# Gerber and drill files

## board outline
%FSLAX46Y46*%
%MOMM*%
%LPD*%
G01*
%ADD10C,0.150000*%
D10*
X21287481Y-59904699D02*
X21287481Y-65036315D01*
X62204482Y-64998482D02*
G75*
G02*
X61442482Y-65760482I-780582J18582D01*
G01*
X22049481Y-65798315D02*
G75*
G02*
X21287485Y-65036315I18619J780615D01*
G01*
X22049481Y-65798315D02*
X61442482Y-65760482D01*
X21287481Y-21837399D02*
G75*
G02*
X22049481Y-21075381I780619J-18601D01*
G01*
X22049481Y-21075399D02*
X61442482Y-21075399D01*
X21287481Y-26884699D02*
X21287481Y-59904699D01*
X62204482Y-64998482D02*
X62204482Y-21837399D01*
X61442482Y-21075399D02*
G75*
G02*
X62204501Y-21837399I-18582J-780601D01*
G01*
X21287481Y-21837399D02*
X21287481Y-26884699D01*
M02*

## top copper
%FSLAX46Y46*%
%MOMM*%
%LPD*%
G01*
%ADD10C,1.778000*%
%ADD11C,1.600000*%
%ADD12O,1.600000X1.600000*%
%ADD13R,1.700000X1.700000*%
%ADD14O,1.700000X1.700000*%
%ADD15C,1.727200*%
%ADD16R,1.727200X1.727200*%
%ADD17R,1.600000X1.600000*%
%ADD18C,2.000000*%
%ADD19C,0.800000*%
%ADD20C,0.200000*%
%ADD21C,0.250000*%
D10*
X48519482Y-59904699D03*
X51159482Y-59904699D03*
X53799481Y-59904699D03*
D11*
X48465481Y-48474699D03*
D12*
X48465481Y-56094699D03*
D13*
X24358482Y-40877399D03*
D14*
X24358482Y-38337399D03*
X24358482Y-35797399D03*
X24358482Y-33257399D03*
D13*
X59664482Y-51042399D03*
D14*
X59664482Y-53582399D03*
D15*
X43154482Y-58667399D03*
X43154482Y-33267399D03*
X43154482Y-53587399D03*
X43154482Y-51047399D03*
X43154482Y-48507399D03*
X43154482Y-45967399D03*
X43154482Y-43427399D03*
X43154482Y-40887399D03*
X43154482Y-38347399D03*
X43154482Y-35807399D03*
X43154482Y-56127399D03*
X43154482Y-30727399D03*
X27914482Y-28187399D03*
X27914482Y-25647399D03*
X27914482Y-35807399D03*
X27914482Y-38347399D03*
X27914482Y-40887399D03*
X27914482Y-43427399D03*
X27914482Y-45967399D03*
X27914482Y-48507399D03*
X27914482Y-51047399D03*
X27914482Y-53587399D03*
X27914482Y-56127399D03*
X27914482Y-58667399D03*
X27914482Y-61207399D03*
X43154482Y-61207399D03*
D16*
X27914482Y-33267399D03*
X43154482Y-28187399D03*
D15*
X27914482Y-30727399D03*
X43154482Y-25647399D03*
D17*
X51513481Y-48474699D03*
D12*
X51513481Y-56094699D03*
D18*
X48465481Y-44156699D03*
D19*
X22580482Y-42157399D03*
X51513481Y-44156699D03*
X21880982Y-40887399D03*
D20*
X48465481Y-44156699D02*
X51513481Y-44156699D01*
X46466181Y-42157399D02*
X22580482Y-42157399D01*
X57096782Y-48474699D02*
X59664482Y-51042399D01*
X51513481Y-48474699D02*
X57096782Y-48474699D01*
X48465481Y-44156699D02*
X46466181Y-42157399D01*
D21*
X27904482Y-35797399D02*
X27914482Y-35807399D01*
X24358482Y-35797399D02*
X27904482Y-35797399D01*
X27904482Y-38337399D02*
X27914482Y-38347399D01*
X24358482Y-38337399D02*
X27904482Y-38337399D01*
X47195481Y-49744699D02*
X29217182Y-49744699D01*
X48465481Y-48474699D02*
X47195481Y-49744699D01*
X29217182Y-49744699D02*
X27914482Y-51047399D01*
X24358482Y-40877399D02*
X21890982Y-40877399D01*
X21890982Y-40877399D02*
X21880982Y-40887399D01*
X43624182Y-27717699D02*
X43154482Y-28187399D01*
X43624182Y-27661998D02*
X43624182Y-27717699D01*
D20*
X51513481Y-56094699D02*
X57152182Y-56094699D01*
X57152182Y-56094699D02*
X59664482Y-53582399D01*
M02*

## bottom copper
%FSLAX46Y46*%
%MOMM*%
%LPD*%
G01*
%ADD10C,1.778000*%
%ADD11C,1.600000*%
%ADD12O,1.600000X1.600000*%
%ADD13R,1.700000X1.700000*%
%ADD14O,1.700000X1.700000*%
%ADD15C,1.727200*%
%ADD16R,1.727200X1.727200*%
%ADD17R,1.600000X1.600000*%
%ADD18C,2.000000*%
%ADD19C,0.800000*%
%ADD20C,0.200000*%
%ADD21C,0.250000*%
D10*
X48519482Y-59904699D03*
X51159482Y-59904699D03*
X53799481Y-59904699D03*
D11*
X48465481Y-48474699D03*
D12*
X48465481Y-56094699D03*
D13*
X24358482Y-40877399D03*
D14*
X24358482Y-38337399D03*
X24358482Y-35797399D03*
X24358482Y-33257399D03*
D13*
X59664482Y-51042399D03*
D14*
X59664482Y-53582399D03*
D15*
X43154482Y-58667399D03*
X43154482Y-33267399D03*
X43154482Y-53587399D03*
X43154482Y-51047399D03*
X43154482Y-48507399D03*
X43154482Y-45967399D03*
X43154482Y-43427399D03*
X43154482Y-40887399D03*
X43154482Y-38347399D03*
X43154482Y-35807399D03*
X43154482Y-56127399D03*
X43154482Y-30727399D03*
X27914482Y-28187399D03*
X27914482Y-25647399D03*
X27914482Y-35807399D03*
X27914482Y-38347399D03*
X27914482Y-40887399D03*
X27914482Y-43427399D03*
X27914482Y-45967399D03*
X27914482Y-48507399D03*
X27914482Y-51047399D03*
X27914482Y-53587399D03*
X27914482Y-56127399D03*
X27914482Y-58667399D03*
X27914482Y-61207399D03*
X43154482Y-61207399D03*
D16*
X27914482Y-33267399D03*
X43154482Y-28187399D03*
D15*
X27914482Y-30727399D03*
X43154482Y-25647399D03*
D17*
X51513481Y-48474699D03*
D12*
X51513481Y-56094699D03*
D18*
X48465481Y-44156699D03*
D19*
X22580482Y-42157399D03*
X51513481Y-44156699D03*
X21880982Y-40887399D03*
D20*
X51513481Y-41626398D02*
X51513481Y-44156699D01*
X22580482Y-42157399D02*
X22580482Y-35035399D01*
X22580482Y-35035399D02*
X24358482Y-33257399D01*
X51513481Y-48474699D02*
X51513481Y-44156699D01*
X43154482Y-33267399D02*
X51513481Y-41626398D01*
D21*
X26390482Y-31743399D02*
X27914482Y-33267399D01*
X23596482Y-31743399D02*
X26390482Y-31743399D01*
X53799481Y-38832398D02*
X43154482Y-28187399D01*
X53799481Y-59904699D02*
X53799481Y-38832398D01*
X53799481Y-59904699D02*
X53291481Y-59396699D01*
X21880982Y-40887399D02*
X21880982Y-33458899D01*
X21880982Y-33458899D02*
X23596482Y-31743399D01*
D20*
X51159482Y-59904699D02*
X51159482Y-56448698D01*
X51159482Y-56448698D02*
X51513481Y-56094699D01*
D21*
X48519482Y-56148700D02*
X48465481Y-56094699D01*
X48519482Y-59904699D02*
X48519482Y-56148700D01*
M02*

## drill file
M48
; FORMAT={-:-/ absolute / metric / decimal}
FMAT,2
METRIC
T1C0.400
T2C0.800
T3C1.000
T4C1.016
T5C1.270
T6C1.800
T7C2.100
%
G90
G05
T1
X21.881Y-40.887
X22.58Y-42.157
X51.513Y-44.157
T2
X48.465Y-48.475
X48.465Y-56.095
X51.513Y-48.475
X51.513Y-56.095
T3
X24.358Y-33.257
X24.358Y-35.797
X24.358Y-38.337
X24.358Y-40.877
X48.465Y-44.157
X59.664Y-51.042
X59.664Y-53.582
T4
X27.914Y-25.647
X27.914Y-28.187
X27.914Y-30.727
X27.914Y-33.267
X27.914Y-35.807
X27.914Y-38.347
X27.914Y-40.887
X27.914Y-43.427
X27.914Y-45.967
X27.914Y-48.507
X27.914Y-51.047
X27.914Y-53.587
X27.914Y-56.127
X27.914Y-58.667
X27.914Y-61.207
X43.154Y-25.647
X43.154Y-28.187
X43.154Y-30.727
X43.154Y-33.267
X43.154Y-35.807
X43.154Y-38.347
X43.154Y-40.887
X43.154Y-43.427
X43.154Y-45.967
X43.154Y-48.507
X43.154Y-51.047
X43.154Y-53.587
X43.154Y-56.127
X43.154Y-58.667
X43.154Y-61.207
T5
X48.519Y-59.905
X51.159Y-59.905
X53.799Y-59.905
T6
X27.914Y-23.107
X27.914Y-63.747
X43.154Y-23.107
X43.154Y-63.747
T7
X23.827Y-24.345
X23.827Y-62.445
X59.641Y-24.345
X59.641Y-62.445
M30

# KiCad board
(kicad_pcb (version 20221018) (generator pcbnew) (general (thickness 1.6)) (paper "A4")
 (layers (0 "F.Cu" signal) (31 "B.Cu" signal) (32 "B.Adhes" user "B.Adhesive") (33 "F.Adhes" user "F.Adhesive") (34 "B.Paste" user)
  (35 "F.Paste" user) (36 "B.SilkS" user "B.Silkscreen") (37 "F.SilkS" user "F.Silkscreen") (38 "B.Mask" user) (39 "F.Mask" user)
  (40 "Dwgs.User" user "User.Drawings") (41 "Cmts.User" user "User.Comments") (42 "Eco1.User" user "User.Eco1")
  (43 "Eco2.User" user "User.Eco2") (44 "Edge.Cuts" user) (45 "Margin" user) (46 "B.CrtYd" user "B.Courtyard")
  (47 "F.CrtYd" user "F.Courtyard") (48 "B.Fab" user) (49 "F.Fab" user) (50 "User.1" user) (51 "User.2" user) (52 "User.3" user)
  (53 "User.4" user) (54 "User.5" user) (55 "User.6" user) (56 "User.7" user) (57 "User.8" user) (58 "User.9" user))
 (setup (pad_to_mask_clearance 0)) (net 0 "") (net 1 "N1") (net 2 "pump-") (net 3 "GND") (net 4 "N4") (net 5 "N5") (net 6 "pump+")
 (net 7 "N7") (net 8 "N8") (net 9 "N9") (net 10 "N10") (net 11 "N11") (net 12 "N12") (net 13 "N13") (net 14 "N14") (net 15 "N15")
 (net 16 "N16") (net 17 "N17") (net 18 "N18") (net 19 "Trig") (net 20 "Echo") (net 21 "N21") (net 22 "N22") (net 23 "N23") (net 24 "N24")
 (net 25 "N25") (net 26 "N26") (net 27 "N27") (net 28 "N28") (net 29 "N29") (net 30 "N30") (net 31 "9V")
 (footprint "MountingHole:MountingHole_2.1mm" (layer "F.Cu") (at 59.641481 62.444699)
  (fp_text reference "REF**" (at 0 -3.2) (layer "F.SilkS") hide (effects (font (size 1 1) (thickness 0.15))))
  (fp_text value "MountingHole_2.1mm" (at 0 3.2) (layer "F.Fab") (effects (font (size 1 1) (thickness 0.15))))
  (pad "" np_thru_hole circle (at 0 0) (size 2.1 2.1) (drill 2.1) (layers "F&B.Cu" "*.Mask")))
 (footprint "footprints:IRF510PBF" (layer "F.Cu") (at 48.519482 59.904699)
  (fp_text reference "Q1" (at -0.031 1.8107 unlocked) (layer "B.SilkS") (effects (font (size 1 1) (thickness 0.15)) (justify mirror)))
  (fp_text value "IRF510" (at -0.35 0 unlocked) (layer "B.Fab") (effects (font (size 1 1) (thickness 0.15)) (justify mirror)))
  (pad "1" thru_hole circle (at 0 0) (size 1.778 1.778) (drill 1.27) (layers "*.Cu" "*.Mask") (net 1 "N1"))
  (pad "2" thru_hole circle (at 2.64 0) (size 1.778 1.778) (drill 1.27) (layers "*.Cu" "*.Mask") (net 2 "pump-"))
  (pad "3" thru_hole circle (at 5.279999 0) (size 1.778 1.778) (drill 1.27) (layers "*.Cu" "*.Mask") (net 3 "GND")))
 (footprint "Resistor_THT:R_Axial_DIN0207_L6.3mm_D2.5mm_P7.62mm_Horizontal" (layer "F.Cu") (at 48.465481 48.474699 -90)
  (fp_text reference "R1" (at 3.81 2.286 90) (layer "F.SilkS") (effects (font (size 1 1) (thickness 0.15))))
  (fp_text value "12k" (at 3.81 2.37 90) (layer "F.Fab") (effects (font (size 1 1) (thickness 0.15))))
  (pad "1" thru_hole circle (at 0 0 270) (size 1.6 1.6) (drill 0.8) (layers "*.Cu" "*.Mask") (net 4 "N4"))
  (pad "2" thru_hole oval (at 7.62 0 270) (size 1.6 1.6) (drill 0.8) (layers "*.Cu" "*.Mask") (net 1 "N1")))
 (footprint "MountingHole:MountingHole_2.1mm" (layer "F.Cu") (at 23.827481 62.444699)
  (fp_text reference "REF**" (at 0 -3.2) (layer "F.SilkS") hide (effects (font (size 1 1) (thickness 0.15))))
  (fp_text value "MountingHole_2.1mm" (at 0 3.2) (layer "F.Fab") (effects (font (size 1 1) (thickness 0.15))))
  (pad "" np_thru_hole circle (at 0 0) (size 2.1 2.1) (drill 2.1) (layers "F&B.Cu" "*.Mask")))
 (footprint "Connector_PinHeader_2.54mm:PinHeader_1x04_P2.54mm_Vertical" (layer "F.Cu") (at 24.358482 40.877399 180)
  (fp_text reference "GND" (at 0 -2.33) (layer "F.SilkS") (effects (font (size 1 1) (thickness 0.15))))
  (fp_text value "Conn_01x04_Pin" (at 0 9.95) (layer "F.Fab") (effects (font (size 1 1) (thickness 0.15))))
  (pad "1" thru_hole rect (at 0 0 180) (size 1.7 1.7) (drill 1) (layers "*.Cu" "*.Mask"))
  (pad "2" thru_hole oval (at 0 2.54 180) (size 1.7 1.7) (drill 1) (layers "*.Cu" "*.Mask"))
  (pad "3" thru_hole oval (at 0 5.08 180) (size 1.7 1.7) (drill 1) (layers "*.Cu" "*.Mask"))
  (pad "4" thru_hole oval (at 0 7.62 180) (size 1.7 1.7) (drill 1) (layers "*.Cu" "*.Mask")))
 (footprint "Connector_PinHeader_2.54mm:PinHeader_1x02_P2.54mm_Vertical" (layer "F.Cu") (at 59.664482 51.042399)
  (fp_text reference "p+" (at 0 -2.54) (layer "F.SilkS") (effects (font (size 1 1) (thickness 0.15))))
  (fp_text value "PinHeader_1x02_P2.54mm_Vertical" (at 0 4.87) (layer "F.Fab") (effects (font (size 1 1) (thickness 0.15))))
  (pad "1" thru_hole rect (at 0 0) (size 1.7 1.7) (drill 1) (layers "*.Cu" "*.Mask"))
  (pad "2" thru_hole oval (at 0 2.54) (size 1.7 1.7) (drill 1) (layers "*.Cu" "*.Mask")))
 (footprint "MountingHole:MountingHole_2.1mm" (layer "F.Cu") (at 59.641481 24.344699)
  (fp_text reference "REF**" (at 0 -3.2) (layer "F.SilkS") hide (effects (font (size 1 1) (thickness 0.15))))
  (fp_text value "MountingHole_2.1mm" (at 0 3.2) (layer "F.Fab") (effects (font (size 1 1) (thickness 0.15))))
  (pad "" np_thru_hole circle (at 0 0) (size 2.1 2.1) (drill 2.1) (layers "F&B.Cu" "*.Mask")))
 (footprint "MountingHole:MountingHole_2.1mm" (layer "F.Cu") (at 23.827481 24.344699)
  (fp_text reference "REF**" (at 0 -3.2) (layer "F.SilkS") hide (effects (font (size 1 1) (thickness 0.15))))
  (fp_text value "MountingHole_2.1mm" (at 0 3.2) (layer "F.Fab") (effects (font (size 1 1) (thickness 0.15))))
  (pad "" np_thru_hole circle (at 0 0) (size 2.1 2.1) (drill 2.1) (layers "F&B.Cu" "*.Mask")))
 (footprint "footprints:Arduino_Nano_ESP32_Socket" (layer "F.Cu") (at 35.534482 65.017399)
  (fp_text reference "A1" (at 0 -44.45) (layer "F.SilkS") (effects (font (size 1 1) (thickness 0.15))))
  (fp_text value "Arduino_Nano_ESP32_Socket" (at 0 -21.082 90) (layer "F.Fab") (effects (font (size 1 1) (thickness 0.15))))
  (pad "" np_thru_hole circle (at -7.62 -41.91) (size 1.8 1.8) (drill 1.8) (layers "F&B.Cu" "*.Mask"))
  (pad "" np_thru_hole circle (at -7.62 -1.27) (size 1.8 1.8) (drill 1.8) (layers "F&B.Cu" "*.Mask"))
  (pad "" np_thru_hole circle (at 7.62 -41.91) (size 1.8 1.8) (drill 1.8) (layers "F&B.Cu" "*.Mask"))
  (pad "" np_thru_hole circle (at 7.62 -1.27) (size 1.8 1.8) (drill 1.8) (layers "F&B.Cu" "*.Mask"))
  (pad "3V3" thru_hole circle (at 7.62 -6.35) (size 1.7272 1.7272) (drill 1.016) (layers "*.Cu" "*.Mask") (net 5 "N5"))
  (pad "5V" thru_hole circle (at 7.62 -31.75) (size 1.7272 1.7272) (drill 1.016) (layers "*.Cu" "*.Mask") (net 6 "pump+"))
  (pad "A0" thru_hole circle (at 7.62 -11.43) (size 1.7272 1.7272) (drill 1.016) (layers "*.Cu" "*.Mask") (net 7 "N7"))
  (pad "A1" thru_hole circle (at 7.62 -13.97) (size 1.7272 1.7272) (drill 1.016) (layers "*.Cu" "*.Mask") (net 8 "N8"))
  (pad "A2" thru_hole circle (at 7.62 -16.51) (size 1.7272 1.7272) (drill 1.016) (layers "*.Cu" "*.Mask") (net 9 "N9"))
  (pad "A3" thru_hole circle (at 7.62 -19.05) (size 1.7272 1.7272) (drill 1.016) (layers "*.Cu" "*.Mask") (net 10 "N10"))
  (pad "A4" thru_hole circle (at 7.62 -21.59) (size 1.7272 1.7272) (drill 1.016) (layers "*.Cu" "*.Mask") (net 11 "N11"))
  (pad "A5" thru_hole circle (at 7.62 -24.13) (size 1.7272 1.7272) (drill 1.016) (layers "*.Cu" "*.Mask") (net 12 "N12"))
  (pad "A6" thru_hole circle (at 7.62 -26.67) (size 1.7272 1.7272) (drill 1.016) (layers "*.Cu" "*.Mask") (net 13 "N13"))
  (pad "A7" thru_hole circle (at 7.62 -29.21) (size 1.7272 1.7272) (drill 1.016) (layers "*.Cu" "*.Mask") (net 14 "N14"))
  (pad "B0" thru_hole circle (at 7.62 -8.89) (size 1.7272 1.7272) (drill 1.016) (layers "*.Cu" "*.Mask") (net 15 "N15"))
  (pad "B1" thru_hole circle (at 7.62 -34.29) (size 1.7272 1.7272) (drill 1.016) (layers "*.Cu" "*.Mask") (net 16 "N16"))
  (pad "D0" thru_hole circle (at -7.62 -36.83) (size 1.7272 1.7272) (drill 1.016) (layers "*.Cu" "*.Mask") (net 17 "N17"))
  (pad "D1" thru_hole circle (at -7.62 -39.37) (size 1.7272 1.7272) (drill 1.016) (layers "*.Cu" "*.Mask") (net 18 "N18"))
  (pad "D2" thru_hole circle (at -7.62 -29.21) (size 1.7272 1.7272) (drill 1.016) (layers "*.Cu" "*.Mask") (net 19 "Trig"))
  (pad "D3" thru_hole circle (at -7.62 -26.67) (size 1.7272 1.7272) (drill 1.016) (layers "*.Cu" "*.Mask") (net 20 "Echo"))
  (pad "D4" thru_hole circle (at -7.62 -24.13) (size 1.7272 1.7272) (drill 1.016) (layers "*.Cu" "*.Mask") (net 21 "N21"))
  (pad "D5" thru_hole circle (at -7.62 -21.59) (size 1.7272 1.7272) (drill 1.016) (layers "*.Cu" "*.Mask") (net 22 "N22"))
  (pad "D6" thru_hole circle (at -7.62 -19.05) (size 1.7272 1.7272) (drill 1.016) (layers "*.Cu" "*.Mask") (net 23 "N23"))
  (pad "D7" thru_hole circle (at -7.62 -16.51) (size 1.7272 1.7272) (drill 1.016) (layers "*.Cu" "*.Mask") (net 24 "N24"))
  (pad "D8" thru_hole circle (at -7.62 -13.97) (size 1.7272 1.7272) (drill 1.016) (layers "*.Cu" "*.Mask") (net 4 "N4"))
  (pad "D9" thru_hole circle (at -7.62 -11.43) (size 1.7272 1.7272) (drill 1.016) (layers "*.Cu" "*.Mask") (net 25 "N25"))
  (pad "D10" thru_hole circle (at -7.62 -8.89) (size 1.7272 1.7272) (drill 1.016) (layers "*.Cu" "*.Mask") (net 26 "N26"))
  (pad "D11" thru_hole circle (at -7.62 -6.35) (size 1.7272 1.7272) (drill 1.016) (layers "*.Cu" "*.Mask") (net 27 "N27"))
  (pad "D12" thru_hole circle (at -7.62 -3.81) (size 1.7272 1.7272) (drill 1.016) (layers "*.Cu" "*.Mask") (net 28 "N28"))
  (pad "D13" thru_hole circle (at 7.62 -3.81) (size 1.7272 1.7272) (drill 1.016) (layers "*.Cu" "*.Mask") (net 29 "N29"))
  (pad "GND1" thru_hole rect (at -7.62 -31.75) (size 1.7272 1.7272) (drill 1.016) (layers "*.Cu" "*.Mask") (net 3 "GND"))
  (pad "GND2" thru_hole rect (at 7.62 -36.83) (size 1.7272 1.7272) (drill 1.016) (layers "*.Cu" "*.Mask") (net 3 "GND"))
  (pad "RST" thru_hole circle (at -7.62 -34.29) (size 1.7272 1.7272) (drill 1.016) (layers "*.Cu" "*.Mask") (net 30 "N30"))
  (pad "VIN" thru_hole circle (at 7.62 -39.37) (size 1.7272 1.7272) (drill 1.016) (layers "*.Cu" "*.Mask") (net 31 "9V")))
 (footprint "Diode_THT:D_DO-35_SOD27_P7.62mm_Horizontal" (layer "F.Cu") (at 51.513481 48.474699 -90)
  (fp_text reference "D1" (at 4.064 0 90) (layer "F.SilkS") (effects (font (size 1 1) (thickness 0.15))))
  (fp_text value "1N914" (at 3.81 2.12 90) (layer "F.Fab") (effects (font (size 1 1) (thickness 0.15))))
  (pad "1" thru_hole rect (at 0 0 270) (size 1.6 1.6) (drill 0.8) (layers "*.Cu" "*.Mask") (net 6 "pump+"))
  (pad "2" thru_hole oval (at 7.62 0 270) (size 1.6 1.6) (drill 0.8) (layers "*.Cu" "*.Mask") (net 2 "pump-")))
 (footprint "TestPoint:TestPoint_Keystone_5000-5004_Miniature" (layer "F.Cu") (at 48.465481 44.156699)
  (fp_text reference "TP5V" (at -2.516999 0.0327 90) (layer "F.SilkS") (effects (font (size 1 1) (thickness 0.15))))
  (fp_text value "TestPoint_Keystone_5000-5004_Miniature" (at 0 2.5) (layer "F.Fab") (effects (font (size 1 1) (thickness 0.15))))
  (pad "1" thru_hole circle (at 0 0) (size 2 2) (drill 1) (layers "*.Cu" "*.Mask")))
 (gr_line (start 21.287481 59.904699) (end 21.287481 65.036315) (stroke (width 0.15) (type default)) (layer "Edge.Cuts"))
 (gr_arc (start 62.204482 64.998482) (mid 61.976015 65.532015) (end 61.442482 65.760482) (stroke (width 0.15) (type default))
  (layer "Edge.Cuts"))
 (gr_arc (start 22.049481 65.798315) (mid 21.515954 65.569842) (end 21.287481 65.036315) (stroke (width 0.15) (type default))
  (layer "Edge.Cuts"))
 (gr_line (start 22.049481 65.798315) (end 61.442482 65.760482) (stroke (width 0.15) (type default)) (layer "Edge.Cuts"))
 (gr_arc (start 21.287481 21.837399) (mid 21.515956 21.303874) (end 22.049481 21.075399) (stroke (width 0.15) (type default))
  (layer "Edge.Cuts"))
 (gr_line (start 22.049481 21.075399) (end 61.442482 21.075399) (stroke (width 0.15) (type default)) (layer "Edge.Cuts"))
 (gr_line (start 21.287481 26.884699) (end 21.287481 59.904699) (stroke (width 0.15) (type default)) (layer "Edge.Cuts"))
 (gr_line (start 62.204482 64.998482) (end 62.204482 21.837399) (stroke (width 0.15) (type default)) (layer "Edge.Cuts"))
 (gr_arc (start 61.442482 21.075399) (mid 61.976006 21.303875) (end 62.204482 21.837399) (stroke (width 0.15) (type default))
  (layer "Edge.Cuts"))
 (gr_line (start 21.287481 21.837399) (end 21.287481 26.884699) (stroke (width 0.15) (type default)) (layer "Edge.Cuts"))
 (segment (start 48.465481 44.156699) (end 51.513481 44.156699) (width 0.2) (layer "F.Cu") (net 6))
 (segment (start 46.466181 42.157399) (end 22.580482 42.157399) (width 0.2) (layer "F.Cu") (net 6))
 (segment (start 57.096782 48.474699) (end 59.664482 51.042399) (width 0.2) (layer "F.Cu") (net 6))
 (segment (start 51.513481 48.474699) (end 57.096782 48.474699) (width 0.2) (layer "F.Cu") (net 6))
 (segment (start 48.465481 44.156699) (end 46.466181 42.157399) (width 0.2) (layer "F.Cu") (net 6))
 (via (at 22.580482 42.157399) (size 0.8) (drill 0.4) (layers "F.Cu" "B.Cu") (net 6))
 (via (at 51.513481 44.156699) (size 0.8) (drill 0.4) (layers "F.Cu" "B.Cu") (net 6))
 (segment (start 51.513481 41.626398) (end 51.513481 44.156699) (width 0.2) (layer "B.Cu") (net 6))
 (segment (start 22.580482 42.157399) (end 22.580482 35.035399) (width 0.2) (layer "B.Cu") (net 6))
 (segment (start 22.580482 35.035399) (end 24.358482 33.257399) (width 0.2) (layer "B.Cu") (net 6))
 (segment (start 51.513481 48.474699) (end 51.513481 44.156699) (width 0.2) (layer "B.Cu") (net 6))
 (segment (start 43.154482 33.267399) (end 51.513481 41.626398) (width 0.2) (layer "B.Cu") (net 6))
 (segment (start 27.904482 35.797399) (end 27.914482 35.807399) (width 0.25) (layer "F.Cu") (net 19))
 (segment (start 24.358482 35.797399) (end 27.904482 35.797399) (width 0.25) (layer "F.Cu") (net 19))
 (segment (start 27.904482 38.337399) (end 27.914482 38.347399) (width 0.25) (layer "F.Cu") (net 20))
 (segment (start 24.358482 38.337399) (end 27.904482 38.337399) (width 0.25) (layer "F.Cu") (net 20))
 (segment (start 47.195481 49.744699) (end 29.217182 49.744699) (width 0.25) (layer "F.Cu") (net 4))
 (segment (start 48.465481 48.474699) (end 47.195481 49.744699) (width 0.25) (layer "F.Cu") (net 4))
 (segment (start 29.217182 49.744699) (end 27.914482 51.047399) (width 0.25) (layer "F.Cu") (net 4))
 (segment (start 24.358482 40.877399) (end 21.890982 40.877399) (width 0.25) (layer "F.Cu") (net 3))
 (segment (start 21.890982 40.877399) (end 21.880982 40.887399) (width 0.25) (layer "F.Cu") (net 3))
 (segment (start 43.624182 27.717699) (end 43.154482 28.187399) (width 0.25) (layer "F.Cu") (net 3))
 (segment (start 43.624182 27.661998) (end 43.624182 27.717699) (width 0.25) (layer "F.Cu") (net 3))
 (via (at 21.880982 40.887399) (size 0.8) (drill 0.4) (layers "F.Cu" "B.Cu") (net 3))
 (segment (start 26.390482 31.743399) (end 27.914482 33.267399) (width 0.25) (layer "B.Cu") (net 3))
 (segment (start 23.596482 31.743399) (end 26.390482 31.743399) (width 0.25) (layer "B.Cu") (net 3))
 (segment (start 53.799481 38.832398) (end 43.154482 28.187399) (width 0.25) (layer "B.Cu") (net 3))
 (segment (start 53.799481 59.904699) (end 53.799481 38.832398) (width 0.25) (layer "B.Cu") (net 3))
 (segment (start 53.799481 59.904699) (end 53.291481 59.396699) (width 0.25) (layer "B.Cu") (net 3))
 (segment (start 21.880982 40.887399) (end 21.880982 33.458899) (width 0.25) (layer "B.Cu") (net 3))
 (segment (start 21.880982 33.458899) (end 23.596482 31.743399) (width 0.25) (layer "B.Cu") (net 3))
 (segment (start 51.513481 56.094699) (end 57.152182 56.094699) (width 0.2) (layer "F.Cu") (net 2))
 (segment (start 57.152182 56.094699) (end 59.664482 53.582399) (width 0.2) (layer "F.Cu") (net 2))
 (segment (start 51.159482 59.904699) (end 51.159482 56.448698) (width 0.2) (layer "B.Cu") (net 2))
 (segment (start 51.159482 56.448698) (end 51.513481 56.094699) (width 0.2) (layer "B.Cu") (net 2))
 (segment (start 48.519482 56.1487) (end 48.465481 56.094699) (width 0.25) (layer "B.Cu") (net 1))
 (segment (start 48.519482 59.904699) (end 48.519482 56.1487) (width 0.25) (layer "B.Cu") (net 1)))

